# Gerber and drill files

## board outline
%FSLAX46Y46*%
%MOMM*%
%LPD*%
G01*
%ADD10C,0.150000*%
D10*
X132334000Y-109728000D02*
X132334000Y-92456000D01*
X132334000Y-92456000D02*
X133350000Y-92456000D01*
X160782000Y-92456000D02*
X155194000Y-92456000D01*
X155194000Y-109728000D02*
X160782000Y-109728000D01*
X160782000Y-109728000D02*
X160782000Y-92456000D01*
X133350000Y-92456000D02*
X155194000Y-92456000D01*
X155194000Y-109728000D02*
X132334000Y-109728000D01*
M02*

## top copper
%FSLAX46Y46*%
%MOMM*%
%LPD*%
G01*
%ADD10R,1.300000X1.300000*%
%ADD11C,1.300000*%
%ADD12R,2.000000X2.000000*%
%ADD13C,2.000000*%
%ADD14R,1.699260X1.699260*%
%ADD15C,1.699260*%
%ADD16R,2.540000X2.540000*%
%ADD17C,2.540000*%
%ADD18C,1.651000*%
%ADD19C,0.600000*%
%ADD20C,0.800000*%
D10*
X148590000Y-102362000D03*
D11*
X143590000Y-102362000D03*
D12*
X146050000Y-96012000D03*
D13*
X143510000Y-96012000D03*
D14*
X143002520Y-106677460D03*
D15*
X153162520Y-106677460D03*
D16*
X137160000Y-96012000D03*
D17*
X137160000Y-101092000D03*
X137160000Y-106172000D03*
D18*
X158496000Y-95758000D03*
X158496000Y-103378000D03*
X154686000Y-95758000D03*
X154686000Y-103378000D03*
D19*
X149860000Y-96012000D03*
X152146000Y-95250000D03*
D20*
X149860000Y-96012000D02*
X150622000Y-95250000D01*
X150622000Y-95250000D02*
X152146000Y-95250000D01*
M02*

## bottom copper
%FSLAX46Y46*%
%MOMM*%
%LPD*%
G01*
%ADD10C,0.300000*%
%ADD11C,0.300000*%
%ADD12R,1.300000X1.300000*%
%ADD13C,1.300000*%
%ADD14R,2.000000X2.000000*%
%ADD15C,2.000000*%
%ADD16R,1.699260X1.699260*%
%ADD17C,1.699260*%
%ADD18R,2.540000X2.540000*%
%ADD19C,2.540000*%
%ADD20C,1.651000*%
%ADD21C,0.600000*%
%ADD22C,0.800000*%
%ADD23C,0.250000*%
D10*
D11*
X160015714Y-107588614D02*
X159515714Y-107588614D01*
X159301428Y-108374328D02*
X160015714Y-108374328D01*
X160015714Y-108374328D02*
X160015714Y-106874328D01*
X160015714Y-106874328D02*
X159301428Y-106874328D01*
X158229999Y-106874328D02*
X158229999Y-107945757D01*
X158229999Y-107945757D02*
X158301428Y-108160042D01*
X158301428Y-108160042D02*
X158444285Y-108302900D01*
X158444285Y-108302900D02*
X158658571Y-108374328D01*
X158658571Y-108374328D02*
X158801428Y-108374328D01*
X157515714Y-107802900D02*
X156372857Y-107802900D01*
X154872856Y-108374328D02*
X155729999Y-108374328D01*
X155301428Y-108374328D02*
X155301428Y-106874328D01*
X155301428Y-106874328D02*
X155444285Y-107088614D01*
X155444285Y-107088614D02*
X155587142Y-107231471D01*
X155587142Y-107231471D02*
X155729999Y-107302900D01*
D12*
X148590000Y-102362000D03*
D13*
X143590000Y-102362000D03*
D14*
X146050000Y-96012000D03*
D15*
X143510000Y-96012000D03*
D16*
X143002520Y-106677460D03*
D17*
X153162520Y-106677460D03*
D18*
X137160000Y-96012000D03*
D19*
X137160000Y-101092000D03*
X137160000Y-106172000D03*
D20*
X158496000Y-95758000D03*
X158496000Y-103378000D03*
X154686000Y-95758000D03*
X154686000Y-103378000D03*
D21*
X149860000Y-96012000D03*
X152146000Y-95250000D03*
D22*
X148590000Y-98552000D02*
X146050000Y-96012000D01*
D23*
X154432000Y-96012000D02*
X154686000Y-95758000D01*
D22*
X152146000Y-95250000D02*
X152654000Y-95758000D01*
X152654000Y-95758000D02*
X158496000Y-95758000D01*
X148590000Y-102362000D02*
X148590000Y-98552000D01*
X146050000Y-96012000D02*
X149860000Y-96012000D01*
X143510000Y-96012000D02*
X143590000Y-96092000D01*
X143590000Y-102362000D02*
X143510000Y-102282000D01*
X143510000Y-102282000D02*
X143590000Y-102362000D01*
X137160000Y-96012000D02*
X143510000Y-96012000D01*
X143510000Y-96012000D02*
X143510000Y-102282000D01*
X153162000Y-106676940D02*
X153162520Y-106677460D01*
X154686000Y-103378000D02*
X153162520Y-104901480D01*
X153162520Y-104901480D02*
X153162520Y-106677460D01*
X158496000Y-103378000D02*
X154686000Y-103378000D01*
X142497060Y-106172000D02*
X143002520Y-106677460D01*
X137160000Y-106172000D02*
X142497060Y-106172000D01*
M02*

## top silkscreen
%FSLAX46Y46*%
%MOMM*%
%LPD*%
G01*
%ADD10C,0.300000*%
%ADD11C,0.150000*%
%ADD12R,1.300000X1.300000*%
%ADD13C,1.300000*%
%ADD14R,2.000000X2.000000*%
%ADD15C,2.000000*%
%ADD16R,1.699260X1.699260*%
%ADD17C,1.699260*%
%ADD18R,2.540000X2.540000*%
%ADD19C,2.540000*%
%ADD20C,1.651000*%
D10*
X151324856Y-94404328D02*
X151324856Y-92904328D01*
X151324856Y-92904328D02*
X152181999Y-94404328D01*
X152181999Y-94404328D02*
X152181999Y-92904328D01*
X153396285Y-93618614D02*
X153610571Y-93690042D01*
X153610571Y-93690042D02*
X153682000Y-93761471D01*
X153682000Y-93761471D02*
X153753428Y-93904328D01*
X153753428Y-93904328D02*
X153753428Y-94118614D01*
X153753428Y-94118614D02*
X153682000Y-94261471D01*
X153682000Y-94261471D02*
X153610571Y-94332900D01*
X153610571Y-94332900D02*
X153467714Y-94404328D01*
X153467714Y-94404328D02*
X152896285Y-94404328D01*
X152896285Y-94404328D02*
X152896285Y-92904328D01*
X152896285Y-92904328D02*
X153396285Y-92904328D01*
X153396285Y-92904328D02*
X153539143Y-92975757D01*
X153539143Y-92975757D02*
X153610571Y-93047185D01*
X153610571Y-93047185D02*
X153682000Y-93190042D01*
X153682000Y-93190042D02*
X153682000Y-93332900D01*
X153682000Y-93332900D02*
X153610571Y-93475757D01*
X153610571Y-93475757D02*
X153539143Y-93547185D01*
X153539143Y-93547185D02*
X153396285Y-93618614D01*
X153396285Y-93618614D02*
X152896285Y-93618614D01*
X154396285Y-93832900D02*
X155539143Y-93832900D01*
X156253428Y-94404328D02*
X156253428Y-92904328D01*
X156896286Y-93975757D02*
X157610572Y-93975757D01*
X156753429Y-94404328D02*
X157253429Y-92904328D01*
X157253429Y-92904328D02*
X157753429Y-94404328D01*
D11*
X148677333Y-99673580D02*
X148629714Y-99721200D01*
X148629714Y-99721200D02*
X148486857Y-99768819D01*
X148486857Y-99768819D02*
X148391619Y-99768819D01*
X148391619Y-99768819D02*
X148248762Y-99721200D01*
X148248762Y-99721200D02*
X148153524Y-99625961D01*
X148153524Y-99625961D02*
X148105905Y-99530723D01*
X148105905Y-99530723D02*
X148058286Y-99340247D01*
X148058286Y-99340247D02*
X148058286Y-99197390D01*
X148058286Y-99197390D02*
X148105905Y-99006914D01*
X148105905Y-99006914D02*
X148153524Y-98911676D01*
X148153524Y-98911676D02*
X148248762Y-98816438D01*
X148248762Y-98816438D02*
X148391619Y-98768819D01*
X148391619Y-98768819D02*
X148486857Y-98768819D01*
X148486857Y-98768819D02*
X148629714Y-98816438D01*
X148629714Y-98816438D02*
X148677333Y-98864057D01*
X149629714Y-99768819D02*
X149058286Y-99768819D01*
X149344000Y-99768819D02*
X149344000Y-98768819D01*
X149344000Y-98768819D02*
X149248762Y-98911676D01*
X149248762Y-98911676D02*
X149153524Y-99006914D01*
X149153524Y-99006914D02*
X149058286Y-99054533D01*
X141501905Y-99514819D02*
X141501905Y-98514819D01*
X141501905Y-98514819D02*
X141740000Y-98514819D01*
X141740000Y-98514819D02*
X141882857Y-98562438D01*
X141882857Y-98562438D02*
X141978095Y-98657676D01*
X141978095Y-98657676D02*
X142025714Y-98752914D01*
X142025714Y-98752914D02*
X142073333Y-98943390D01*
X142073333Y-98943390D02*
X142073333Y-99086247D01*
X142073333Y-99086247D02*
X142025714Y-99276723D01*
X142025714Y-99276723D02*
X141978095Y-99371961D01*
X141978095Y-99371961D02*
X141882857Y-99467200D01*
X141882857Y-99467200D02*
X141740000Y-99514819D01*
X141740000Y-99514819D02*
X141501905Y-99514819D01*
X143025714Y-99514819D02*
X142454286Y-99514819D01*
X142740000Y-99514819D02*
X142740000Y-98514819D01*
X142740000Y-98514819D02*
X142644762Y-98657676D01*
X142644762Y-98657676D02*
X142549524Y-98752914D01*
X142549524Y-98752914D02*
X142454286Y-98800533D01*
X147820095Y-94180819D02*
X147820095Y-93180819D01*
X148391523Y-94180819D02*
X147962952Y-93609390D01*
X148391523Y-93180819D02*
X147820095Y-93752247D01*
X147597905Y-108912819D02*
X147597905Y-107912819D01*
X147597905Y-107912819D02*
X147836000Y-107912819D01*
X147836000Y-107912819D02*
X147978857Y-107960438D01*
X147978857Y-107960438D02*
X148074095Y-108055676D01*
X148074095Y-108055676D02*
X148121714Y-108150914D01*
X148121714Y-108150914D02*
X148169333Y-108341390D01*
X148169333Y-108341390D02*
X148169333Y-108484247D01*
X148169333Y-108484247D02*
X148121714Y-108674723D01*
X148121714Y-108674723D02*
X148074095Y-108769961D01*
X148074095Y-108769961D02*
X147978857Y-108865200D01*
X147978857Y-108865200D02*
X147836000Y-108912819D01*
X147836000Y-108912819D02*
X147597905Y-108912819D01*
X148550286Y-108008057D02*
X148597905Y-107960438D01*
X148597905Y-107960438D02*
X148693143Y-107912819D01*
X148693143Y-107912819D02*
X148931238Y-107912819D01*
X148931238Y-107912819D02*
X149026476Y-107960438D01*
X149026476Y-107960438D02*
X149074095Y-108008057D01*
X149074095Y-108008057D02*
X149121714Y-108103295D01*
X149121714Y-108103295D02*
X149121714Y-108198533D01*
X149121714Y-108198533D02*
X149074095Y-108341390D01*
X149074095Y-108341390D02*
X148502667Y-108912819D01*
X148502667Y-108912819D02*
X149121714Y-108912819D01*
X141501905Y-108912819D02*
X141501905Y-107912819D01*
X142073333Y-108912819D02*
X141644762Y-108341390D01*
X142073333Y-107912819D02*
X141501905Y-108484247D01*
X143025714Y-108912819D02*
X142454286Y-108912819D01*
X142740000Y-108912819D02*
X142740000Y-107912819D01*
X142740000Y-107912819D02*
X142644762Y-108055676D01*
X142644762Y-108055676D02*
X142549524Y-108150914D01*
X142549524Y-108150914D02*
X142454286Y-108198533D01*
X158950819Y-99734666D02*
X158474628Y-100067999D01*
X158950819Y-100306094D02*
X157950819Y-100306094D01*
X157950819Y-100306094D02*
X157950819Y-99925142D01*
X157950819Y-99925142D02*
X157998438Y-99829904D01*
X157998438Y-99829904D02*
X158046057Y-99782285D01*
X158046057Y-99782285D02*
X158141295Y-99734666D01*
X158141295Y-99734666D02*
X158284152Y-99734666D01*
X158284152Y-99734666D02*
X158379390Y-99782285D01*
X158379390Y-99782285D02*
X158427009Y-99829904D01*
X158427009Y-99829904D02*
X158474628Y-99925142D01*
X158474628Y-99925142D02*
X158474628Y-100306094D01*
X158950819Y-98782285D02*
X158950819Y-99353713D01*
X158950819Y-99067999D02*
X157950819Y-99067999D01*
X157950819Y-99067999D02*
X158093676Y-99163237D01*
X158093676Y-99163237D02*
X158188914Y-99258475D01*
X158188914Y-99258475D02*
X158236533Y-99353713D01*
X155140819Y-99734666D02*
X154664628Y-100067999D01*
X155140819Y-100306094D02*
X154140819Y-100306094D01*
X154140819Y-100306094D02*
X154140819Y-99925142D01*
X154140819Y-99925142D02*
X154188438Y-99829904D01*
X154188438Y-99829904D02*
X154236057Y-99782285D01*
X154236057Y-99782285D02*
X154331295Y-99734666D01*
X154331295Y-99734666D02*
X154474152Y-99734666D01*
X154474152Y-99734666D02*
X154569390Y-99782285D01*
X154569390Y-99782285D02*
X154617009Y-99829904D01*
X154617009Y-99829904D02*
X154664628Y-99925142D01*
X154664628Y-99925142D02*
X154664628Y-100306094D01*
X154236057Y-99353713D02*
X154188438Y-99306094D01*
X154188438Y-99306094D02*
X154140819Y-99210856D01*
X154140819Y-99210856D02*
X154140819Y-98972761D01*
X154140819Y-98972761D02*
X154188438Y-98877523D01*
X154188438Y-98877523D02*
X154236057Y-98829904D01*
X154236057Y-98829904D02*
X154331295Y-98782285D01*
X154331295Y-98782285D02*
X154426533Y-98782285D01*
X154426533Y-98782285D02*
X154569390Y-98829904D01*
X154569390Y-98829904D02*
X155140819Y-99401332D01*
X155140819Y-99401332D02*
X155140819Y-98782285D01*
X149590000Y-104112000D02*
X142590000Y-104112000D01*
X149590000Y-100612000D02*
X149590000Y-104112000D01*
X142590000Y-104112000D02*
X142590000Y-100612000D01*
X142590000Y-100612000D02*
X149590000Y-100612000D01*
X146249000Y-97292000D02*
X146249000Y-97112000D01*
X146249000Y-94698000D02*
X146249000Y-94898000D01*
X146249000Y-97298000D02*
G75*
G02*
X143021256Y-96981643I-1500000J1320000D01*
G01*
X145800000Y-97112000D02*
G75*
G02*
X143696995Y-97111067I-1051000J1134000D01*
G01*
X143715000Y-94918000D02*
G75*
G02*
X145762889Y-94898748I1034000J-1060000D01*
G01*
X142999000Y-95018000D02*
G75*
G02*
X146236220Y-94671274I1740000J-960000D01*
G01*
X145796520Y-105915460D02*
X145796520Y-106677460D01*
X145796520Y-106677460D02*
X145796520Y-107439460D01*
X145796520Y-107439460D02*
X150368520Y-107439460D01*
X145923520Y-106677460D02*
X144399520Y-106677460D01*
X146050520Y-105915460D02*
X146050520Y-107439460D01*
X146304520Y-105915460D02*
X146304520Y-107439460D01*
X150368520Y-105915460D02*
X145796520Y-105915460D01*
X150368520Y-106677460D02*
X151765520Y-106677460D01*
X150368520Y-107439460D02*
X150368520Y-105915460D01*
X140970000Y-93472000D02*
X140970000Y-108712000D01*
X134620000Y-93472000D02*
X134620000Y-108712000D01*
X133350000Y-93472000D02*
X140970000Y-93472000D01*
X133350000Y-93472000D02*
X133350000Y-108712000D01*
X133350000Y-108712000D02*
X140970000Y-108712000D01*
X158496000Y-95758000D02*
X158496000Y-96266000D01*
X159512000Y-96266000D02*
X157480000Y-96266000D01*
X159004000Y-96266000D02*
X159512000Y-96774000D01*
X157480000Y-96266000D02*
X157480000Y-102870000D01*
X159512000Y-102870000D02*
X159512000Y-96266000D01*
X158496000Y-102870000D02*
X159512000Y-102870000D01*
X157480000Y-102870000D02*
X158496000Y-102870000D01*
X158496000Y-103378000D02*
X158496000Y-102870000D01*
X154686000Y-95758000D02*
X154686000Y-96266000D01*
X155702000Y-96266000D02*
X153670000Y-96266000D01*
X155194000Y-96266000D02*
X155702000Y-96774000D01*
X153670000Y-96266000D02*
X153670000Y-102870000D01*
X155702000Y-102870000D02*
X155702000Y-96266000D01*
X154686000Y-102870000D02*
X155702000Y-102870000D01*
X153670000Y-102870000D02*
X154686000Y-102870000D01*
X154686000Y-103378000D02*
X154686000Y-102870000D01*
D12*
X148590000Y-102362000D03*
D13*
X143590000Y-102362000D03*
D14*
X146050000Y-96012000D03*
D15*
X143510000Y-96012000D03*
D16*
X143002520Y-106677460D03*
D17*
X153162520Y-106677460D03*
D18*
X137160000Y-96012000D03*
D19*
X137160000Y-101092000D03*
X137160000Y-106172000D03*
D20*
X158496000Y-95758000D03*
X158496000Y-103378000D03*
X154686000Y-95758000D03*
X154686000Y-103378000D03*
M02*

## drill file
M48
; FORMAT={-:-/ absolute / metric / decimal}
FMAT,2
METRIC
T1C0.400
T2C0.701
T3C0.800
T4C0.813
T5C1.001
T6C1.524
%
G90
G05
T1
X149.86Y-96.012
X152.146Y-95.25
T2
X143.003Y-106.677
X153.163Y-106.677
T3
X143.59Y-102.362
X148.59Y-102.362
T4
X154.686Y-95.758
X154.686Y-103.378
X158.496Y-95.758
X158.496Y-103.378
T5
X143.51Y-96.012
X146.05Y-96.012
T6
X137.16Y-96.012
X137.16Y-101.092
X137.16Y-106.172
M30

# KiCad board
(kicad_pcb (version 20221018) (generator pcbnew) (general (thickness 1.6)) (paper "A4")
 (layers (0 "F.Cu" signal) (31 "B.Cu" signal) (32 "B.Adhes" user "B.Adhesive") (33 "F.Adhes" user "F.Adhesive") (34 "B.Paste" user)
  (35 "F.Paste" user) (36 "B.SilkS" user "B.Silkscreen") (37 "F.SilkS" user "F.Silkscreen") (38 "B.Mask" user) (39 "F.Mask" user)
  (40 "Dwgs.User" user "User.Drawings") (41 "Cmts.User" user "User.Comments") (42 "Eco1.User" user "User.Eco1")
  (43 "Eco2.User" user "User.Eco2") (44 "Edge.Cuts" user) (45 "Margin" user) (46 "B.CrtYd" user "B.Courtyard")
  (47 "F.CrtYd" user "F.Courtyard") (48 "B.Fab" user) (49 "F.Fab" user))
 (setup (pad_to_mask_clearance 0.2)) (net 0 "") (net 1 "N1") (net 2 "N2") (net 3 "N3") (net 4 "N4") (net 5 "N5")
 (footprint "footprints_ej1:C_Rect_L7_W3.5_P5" (layer "F.Cu") (at 148.59 102.362 180)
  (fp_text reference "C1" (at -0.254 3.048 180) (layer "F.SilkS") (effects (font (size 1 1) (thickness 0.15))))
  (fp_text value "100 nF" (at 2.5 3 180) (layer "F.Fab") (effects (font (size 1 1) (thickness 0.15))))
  (fp_line (start -1 -1.75) (end 6 -1.75) (stroke (width 0.15) (type solid)) (layer "F.SilkS"))
  (fp_line (start -1 1.75) (end -1 -1.75) (stroke (width 0.15) (type solid)) (layer "F.SilkS"))
  (fp_line (start 6 -1.75) (end 6 1.75) (stroke (width 0.15) (type solid)) (layer "F.SilkS"))
  (fp_line (start 6 1.75) (end -1 1.75) (stroke (width 0.15) (type solid)) (layer "F.SilkS"))
  (pad "1" thru_hole rect (at 0 0 180) (size 1.3 1.3) (drill 0.8) (layers "*.Cu" "*.Mask" "F.SilkS") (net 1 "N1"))
  (pad "2" thru_hole circle (at 5 0 180) (size 1.3 1.3) (drill 0.8) (layers "*.Cu" "*.Mask" "F.SilkS") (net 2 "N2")))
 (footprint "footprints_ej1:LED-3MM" (layer "F.Cu") (at 146.05 96.012 180)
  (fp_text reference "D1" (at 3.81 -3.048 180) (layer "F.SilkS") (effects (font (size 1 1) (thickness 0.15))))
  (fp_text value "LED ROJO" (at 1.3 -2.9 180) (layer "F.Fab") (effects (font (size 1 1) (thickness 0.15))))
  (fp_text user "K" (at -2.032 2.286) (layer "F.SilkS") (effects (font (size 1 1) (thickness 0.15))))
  (fp_line (start -0.199 -1.28) (end -0.199 -1.1) (stroke (width 0.15) (type solid)) (layer "F.SilkS"))
  (fp_line (start -0.199 1.314) (end -0.199 1.114) (stroke (width 0.15) (type solid)) (layer "F.SilkS"))
  (fp_arc (start -0.199 -1.286) (mid 1.495903 -1.954571) (end 3.028744 -0.969643) (stroke (width 0.15) (type solid)) (layer "F.SilkS"))
  (fp_arc (start 0.25 -1.1) (mid 1.301686 -1.512142) (end 2.353005 -1.099067) (stroke (width 0.15) (type solid)) (layer "F.SilkS"))
  (fp_arc (start 2.335 1.094) (mid 1.31492 1.51473) (end 0.287111 1.113252) (stroke (width 0.15) (type solid)) (layer "F.SilkS"))
  (fp_arc (start 3.051 0.994) (mid 1.522637 2.009958) (end -0.18622 1.340726) (stroke (width 0.15) (type solid)) (layer "F.SilkS"))
  (pad "1" thru_hole rect (at 0 0 270) (size 2 2) (drill 1.00076) (layers "*.Cu" "*.Mask" "F.SilkS") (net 1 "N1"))
  (pad "2" thru_hole circle (at 2.54 0 180) (size 2 2) (drill 1.00076) (layers "*.Cu" "*.Mask" "F.SilkS") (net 2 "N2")))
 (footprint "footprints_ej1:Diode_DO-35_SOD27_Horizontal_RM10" (layer "F.Cu") (at 143.002 106.68)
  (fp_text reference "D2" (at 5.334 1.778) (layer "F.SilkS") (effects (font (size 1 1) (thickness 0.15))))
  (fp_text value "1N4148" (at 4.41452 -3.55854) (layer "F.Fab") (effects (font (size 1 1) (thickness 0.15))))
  (fp_line (start 2.79452 -0.76454) (end 2.79452 -0.00254) (stroke (width 0.15) (type solid)) (layer "F.SilkS"))
  (fp_line (start 2.79452 -0.00254) (end 2.79452 0.75946) (stroke (width 0.15) (type solid)) (layer "F.SilkS"))
  (fp_line (start 2.79452 0.75946) (end 7.36652 0.75946) (stroke (width 0.15) (type solid)) (layer "F.SilkS"))
  (fp_line (start 2.92152 -0.00254) (end 1.39752 -0.00254) (stroke (width 0.15) (type solid)) (layer "F.SilkS"))
  (fp_line (start 3.04852 -0.76454) (end 3.04852 0.75946) (stroke (width 0.15) (type solid)) (layer "F.SilkS"))
  (fp_line (start 3.30252 -0.76454) (end 3.30252 0.75946) (stroke (width 0.15) (type solid)) (layer "F.SilkS"))
  (fp_line (start 7.36652 -0.76454) (end 2.79452 -0.76454) (stroke (width 0.15) (type solid)) (layer "F.SilkS"))
  (fp_line (start 7.36652 -0.00254) (end 8.76352 -0.00254) (stroke (width 0.15) (type solid)) (layer "F.SilkS"))
  (fp_line (start 7.36652 0.75946) (end 7.36652 -0.76454) (stroke (width 0.15) (type solid)) (layer "F.SilkS"))
  (pad "1" thru_hole rect (at 0.00052 -0.00254 180) (size 1.69926 1.69926) (drill 0.70104) (layers "*.Cu" "*.Mask" "F.SilkS") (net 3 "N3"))
  (pad "2" thru_hole circle (at 10.16052 -0.00254 180) (size 1.69926 1.69926) (drill 0.70104) (layers "*.Cu" "*.Mask" "F.SilkS")
   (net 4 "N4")))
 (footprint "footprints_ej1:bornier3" (layer "F.Cu") (at 137.16 101.092 -90)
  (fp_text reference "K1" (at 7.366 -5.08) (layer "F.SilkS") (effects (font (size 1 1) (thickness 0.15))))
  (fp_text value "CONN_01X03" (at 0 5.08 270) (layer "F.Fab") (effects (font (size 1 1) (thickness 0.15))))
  (fp_line (start -7.62 -3.81) (end 7.62 -3.81) (stroke (width 0.15) (type solid)) (layer "F.SilkS"))
  (fp_line (start -7.62 2.54) (end 7.62 2.54) (stroke (width 0.15) (type solid)) (layer "F.SilkS"))
  (fp_line (start -7.62 3.81) (end -7.62 -3.81) (stroke (width 0.15) (type solid)) (layer "F.SilkS"))
  (fp_line (start -7.62 3.81) (end 7.62 3.81) (stroke (width 0.15) (type solid)) (layer "F.SilkS"))
  (fp_line (start 7.62 3.81) (end 7.62 -3.81) (stroke (width 0.15) (type solid)) (layer "F.SilkS"))
  (pad "1" thru_hole rect (at -5.08 0 270) (size 2.54 2.54) (drill 1.524) (layers "*.Cu" "*.Mask" "F.SilkS") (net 2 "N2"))
  (pad "2" thru_hole circle (at 0 0 270) (size 2.54 2.54) (drill 1.524) (layers "*.Cu" "*.Mask" "F.SilkS") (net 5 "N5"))
  (pad "3" thru_hole circle (at 5.08 0 270) (size 2.54 2.54) (drill 1.524) (layers "*.Cu" "*.Mask" "F.SilkS") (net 3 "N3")))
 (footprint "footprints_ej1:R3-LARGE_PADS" (layer "F.Cu") (at 158.496 99.568 -90)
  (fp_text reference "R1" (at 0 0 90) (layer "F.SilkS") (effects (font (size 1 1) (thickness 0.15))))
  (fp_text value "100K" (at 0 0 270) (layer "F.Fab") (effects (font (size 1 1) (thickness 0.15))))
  (fp_line (start -3.81 0) (end -3.302 0) (stroke (width 0.15) (type solid)) (layer "F.SilkS"))
  (fp_line (start -3.302 -1.016) (end -3.302 1.016) (stroke (width 0.15) (type solid)) (layer "F.SilkS"))
  (fp_line (start -3.302 -0.508) (end -2.794 -1.016) (stroke (width 0.15) (type solid)) (layer "F.SilkS"))
  (fp_line (start -3.302 1.016) (end 3.302 1.016) (stroke (width 0.15) (type solid)) (layer "F.SilkS"))
  (fp_line (start 3.302 -1.016) (end -3.302 -1.016) (stroke (width 0.15) (type solid)) (layer "F.SilkS"))
  (fp_line (start 3.302 0) (end 3.302 -1.016) (stroke (width 0.15) (type solid)) (layer "F.SilkS"))
  (fp_line (start 3.302 1.016) (end 3.302 0) (stroke (width 0.15) (type solid)) (layer "F.SilkS"))
  (fp_line (start 3.81 0) (end 3.302 0) (stroke (width 0.15) (type solid)) (layer "F.SilkS"))
  (pad "1" thru_hole circle (at -3.81 0 270) (size 1.651 1.651) (drill 0.8128) (layers "*.Cu" "*.Mask" "F.SilkS") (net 1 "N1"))
  (pad "2" thru_hole circle (at 3.81 0 270) (size 1.651 1.651) (drill 0.8128) (layers "*.Cu" "*.Mask" "F.SilkS") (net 4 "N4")))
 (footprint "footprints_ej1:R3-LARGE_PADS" (layer "F.Cu") (at 154.686 99.568 -90)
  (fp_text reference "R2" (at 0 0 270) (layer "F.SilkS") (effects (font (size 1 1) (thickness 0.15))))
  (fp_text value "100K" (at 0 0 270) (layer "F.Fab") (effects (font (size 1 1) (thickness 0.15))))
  (fp_line (start -3.81 0) (end -3.302 0) (stroke (width 0.15) (type solid)) (layer "F.SilkS"))
  (fp_line (start -3.302 -1.016) (end -3.302 1.016) (stroke (width 0.15) (type solid)) (layer "F.SilkS"))
  (fp_line (start -3.302 -0.508) (end -2.794 -1.016) (stroke (width 0.15) (type solid)) (layer "F.SilkS"))
  (fp_line (start -3.302 1.016) (end 3.302 1.016) (stroke (width 0.15) (type solid)) (layer "F.SilkS"))
  (fp_line (start 3.302 -1.016) (end -3.302 -1.016) (stroke (width 0.15) (type solid)) (layer "F.SilkS"))
  (fp_line (start 3.302 0) (end 3.302 -1.016) (stroke (width 0.15) (type solid)) (layer "F.SilkS"))
  (fp_line (start 3.302 1.016) (end 3.302 0) (stroke (width 0.15) (type solid)) (layer "F.SilkS"))
  (fp_line (start 3.81 0) (end 3.302 0) (stroke (width 0.15) (type solid)) (layer "F.SilkS"))
  (pad "1" thru_hole circle (at -3.81 0 270) (size 1.651 1.651) (drill 0.8128) (layers "*.Cu" "*.Mask" "F.SilkS") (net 1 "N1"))
  (pad "2" thru_hole circle (at 3.81 0 270) (size 1.651 1.651) (drill 0.8128) (layers "*.Cu" "*.Mask" "F.SilkS") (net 4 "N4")))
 (gr_line (start 132.334 109.728) (end 132.334 92.456) (stroke (width 0.15) (type solid)) (layer "Edge.Cuts"))
 (gr_line (start 132.334 92.456) (end 133.35 92.456) (stroke (width 0.15) (type solid)) (layer "Edge.Cuts"))
 (gr_line (start 160.782 92.456) (end 155.194 92.456) (stroke (width 0.15) (type solid)) (layer "Edge.Cuts"))
 (gr_line (start 155.194 109.728) (end 160.782 109.728) (stroke (width 0.15) (type solid)) (layer "Edge.Cuts"))
 (gr_line (start 160.782 109.728) (end 160.782 92.456) (stroke (width 0.15) (type solid)) (layer "Edge.Cuts"))
 (gr_line (start 133.35 92.456) (end 155.194 92.456) (stroke (width 0.15) (type solid)) (layer "Edge.Cuts"))
 (gr_line (start 155.194 109.728) (end 132.334 109.728) (stroke (width 0.15) (type solid)) (layer "Edge.Cuts"))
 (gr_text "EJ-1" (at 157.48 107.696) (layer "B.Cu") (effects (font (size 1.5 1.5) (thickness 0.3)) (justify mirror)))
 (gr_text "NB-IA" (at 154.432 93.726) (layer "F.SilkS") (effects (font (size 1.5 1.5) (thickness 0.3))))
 (segment (start 149.86 96.012) (end 150.622 95.25) (width 0.8) (layer "F.Cu") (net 1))
 (segment (start 150.622 95.25) (end 152.146 95.25) (width 0.8) (layer "F.Cu") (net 1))
 (via (at 149.86 96.012) (size 0.6) (drill 0.4) (layers "F.Cu" "B.Cu") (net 1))
 (via (at 152.146 95.25) (size 0.6) (drill 0.4) (layers "F.Cu" "B.Cu") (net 1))
 (segment (start 148.59 98.552) (end 146.05 96.012) (width 0.8) (layer "B.Cu") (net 1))
 (segment (start 154.432 96.012) (end 154.686 95.758) (width 0.25) (layer "B.Cu") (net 1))
 (segment (start 152.146 95.25) (end 152.654 95.758) (width 0.8) (layer "B.Cu") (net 1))
 (segment (start 152.654 95.758) (end 158.496 95.758) (width 0.8) (layer "B.Cu") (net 1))
 (segment (start 148.59 102.362) (end 148.59 98.552) (width 0.8) (layer "B.Cu") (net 1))
 (segment (start 146.05 96.012) (end 149.86 96.012) (width 0.8) (layer "B.Cu") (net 1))
 (segment (start 143.51 96.012) (end 143.59 96.092) (width 0.8) (layer "B.Cu") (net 2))
 (segment (start 143.59 102.362) (end 143.51 102.282) (width 0.8) (layer "B.Cu") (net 2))
 (segment (start 143.51 102.282) (end 143.59 102.362) (width 0.8) (layer "B.Cu") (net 2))
 (segment (start 137.16 96.012) (end 143.51 96.012) (width 0.8) (layer "B.Cu") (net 2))
 (segment (start 143.51 96.012) (end 143.51 102.282) (width 0.8) (layer "B.Cu") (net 2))
 (segment (start 153.162 106.67694) (end 153.16252 106.67746) (width 0.8) (layer "B.Cu") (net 4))
 (segment (start 154.686 103.378) (end 153.16252 104.90148) (width 0.8) (layer "B.Cu") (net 4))
 (segment (start 153.16252 104.90148) (end 153.16252 106.67746) (width 0.8) (layer "B.Cu") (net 4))
 (segment (start 158.496 103.378) (end 154.686 103.378) (width 0.8) (layer "B.Cu") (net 4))
 (segment (start 142.49706 106.172) (end 143.00252 106.67746) (width 0.8) (layer "B.Cu") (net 3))
 (segment (start 137.16 106.172) (end 142.49706 106.172) (width 0.8) (layer "B.Cu") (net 3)))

